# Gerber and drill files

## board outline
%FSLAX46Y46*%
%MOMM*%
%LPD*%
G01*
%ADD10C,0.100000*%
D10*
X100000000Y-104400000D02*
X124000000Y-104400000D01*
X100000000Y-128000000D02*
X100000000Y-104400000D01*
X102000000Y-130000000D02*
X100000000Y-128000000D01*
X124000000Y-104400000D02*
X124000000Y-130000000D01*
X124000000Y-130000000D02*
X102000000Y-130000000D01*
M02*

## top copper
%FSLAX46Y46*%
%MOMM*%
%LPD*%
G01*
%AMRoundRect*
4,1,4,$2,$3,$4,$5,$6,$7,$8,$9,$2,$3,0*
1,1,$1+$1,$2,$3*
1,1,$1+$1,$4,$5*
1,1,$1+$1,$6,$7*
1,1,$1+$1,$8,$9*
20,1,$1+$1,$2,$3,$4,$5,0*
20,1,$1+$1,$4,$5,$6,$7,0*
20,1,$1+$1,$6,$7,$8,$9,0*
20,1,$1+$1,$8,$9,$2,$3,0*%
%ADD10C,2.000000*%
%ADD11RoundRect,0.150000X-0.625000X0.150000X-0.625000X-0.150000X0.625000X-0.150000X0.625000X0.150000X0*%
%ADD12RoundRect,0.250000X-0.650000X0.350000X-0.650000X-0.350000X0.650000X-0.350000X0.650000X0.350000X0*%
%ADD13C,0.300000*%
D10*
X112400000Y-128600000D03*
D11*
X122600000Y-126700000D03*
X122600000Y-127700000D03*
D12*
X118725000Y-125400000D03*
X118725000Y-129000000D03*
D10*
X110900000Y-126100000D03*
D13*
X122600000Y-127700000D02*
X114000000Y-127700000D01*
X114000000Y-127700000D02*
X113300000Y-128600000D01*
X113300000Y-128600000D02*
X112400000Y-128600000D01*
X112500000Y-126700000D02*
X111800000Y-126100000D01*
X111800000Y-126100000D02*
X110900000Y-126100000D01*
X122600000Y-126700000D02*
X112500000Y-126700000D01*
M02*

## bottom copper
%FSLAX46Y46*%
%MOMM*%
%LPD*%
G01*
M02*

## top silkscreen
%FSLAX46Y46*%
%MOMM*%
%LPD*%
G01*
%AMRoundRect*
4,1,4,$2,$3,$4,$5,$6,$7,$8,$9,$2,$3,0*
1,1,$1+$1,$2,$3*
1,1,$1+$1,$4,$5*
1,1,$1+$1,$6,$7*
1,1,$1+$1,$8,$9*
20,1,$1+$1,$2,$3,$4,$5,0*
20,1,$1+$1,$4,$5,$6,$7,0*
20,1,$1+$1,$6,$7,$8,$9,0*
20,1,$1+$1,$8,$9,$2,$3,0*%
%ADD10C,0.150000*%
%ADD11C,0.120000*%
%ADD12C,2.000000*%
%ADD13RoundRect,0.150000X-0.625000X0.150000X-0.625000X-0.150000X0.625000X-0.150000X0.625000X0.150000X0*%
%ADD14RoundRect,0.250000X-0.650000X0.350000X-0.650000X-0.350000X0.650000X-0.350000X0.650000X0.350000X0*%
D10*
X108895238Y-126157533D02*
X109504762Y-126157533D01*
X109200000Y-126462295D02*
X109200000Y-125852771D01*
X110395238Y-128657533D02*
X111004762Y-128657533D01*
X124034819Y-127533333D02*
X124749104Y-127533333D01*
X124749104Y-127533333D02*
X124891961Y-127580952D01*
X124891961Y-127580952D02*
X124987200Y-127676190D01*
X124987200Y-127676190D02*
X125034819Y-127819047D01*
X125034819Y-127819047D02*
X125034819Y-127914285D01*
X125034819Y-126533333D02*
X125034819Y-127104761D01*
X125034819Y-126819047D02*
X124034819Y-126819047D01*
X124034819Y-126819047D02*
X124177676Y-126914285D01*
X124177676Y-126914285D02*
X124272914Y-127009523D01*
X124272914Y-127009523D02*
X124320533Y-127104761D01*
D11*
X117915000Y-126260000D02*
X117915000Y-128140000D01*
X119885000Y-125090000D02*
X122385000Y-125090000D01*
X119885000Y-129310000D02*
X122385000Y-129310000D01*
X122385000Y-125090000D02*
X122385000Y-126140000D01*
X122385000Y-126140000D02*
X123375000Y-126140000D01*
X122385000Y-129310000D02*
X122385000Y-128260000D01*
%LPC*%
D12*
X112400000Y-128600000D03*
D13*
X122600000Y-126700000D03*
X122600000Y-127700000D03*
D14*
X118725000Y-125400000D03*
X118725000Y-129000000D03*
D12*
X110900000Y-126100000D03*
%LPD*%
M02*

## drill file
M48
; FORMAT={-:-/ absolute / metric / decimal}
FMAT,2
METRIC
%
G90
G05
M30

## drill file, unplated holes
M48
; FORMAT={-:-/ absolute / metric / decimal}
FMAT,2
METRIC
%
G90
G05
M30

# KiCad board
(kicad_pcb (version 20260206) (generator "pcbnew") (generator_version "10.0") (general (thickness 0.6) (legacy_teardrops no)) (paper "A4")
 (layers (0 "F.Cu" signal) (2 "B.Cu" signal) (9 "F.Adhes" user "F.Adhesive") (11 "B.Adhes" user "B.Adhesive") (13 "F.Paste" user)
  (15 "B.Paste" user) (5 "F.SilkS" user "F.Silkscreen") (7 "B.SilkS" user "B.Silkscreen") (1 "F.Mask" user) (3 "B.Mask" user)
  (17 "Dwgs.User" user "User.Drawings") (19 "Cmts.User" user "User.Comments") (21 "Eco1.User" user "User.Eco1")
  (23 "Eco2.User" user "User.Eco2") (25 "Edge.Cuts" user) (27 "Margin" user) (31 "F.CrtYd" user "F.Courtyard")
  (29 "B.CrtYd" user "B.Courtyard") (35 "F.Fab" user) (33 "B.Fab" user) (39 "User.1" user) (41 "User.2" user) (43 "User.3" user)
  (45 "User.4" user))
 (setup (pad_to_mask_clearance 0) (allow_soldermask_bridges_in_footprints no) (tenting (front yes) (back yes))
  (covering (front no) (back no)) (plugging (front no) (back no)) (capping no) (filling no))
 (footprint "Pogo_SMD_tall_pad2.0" (layer "F.Cu") (at 112.4 128.6)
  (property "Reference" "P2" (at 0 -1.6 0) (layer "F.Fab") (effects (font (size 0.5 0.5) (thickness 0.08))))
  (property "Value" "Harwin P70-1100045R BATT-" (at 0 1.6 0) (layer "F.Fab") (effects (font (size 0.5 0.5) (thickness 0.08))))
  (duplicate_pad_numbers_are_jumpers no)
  (pad "1" smd circle (at 0 0) (size 2 2) (layers "F.Cu" "F.Mask" "F.Paste") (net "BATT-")))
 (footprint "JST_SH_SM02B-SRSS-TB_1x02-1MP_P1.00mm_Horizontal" (layer "F.Cu") (at 120.6 127.2 -90)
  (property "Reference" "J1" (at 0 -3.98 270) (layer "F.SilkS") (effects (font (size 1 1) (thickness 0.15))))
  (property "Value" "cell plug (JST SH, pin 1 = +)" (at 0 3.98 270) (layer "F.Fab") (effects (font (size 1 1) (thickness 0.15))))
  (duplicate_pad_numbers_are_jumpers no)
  (fp_line (start -0.94 2.685) (end 0.94 2.685) (stroke (width 0.12) (type solid)) (layer "F.SilkS"))
  (fp_line (start -2.11 0.715) (end -2.11 -1.785) (stroke (width 0.12) (type solid)) (layer "F.SilkS"))
  (fp_line (start 2.11 0.715) (end 2.11 -1.785) (stroke (width 0.12) (type solid)) (layer "F.SilkS"))
  (fp_line (start -2.11 -1.785) (end -1.06 -1.785) (stroke (width 0.12) (type solid)) (layer "F.SilkS"))
  (fp_line (start -1.06 -1.785) (end -1.06 -2.775) (stroke (width 0.12) (type solid)) (layer "F.SilkS"))
  (fp_line (start 2.11 -1.785) (end 1.06 -1.785) (stroke (width 0.12) (type solid)) (layer "F.SilkS"))
  (pad "1" smd roundrect (at -0.5 -2 270) (size 0.6 1.55) (layers "F.Cu" "F.Mask" "F.Paste") (roundrect_rratio 0.25) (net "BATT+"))
  (pad "2" smd roundrect (at 0.5 -2 270) (size 0.6 1.55) (layers "F.Cu" "F.Mask" "F.Paste") (roundrect_rratio 0.25) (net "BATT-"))
  (pad "MP" smd roundrect (at -1.8 1.875 270) (size 1.2 1.8) (layers "F.Cu" "F.Mask" "F.Paste") (roundrect_rratio 0.208333))
  (pad "MP" smd roundrect (at 1.8 1.875 270) (size 1.2 1.8) (layers "F.Cu" "F.Mask" "F.Paste") (roundrect_rratio 0.208333)))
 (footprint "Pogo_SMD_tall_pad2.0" (layer "F.Cu") (at 110.9 126.1)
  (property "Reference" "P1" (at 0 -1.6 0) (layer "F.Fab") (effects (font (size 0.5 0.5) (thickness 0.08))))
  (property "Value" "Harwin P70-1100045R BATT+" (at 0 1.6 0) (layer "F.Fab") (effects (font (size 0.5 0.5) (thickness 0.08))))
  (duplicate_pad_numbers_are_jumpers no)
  (pad "1" smd circle (at 0 0) (size 2 2) (layers "F.Cu" "F.Mask" "F.Paste") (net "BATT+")))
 (gr_line (start 100 104.4) (end 124 104.4) (stroke (width 0.1) (type default)) (layer "Edge.Cuts"))
 (gr_line (start 100 128) (end 100 104.4) (stroke (width 0.1) (type default)) (layer "Edge.Cuts"))
 (gr_line (start 102 130) (end 100 128) (stroke (width 0.1) (type default)) (layer "Edge.Cuts"))
 (gr_line (start 124 104.4) (end 124 130) (stroke (width 0.1) (type default)) (layer "Edge.Cuts"))
 (gr_line (start 124 130) (end 102 130) (stroke (width 0.1) (type default)) (layer "Edge.Cuts"))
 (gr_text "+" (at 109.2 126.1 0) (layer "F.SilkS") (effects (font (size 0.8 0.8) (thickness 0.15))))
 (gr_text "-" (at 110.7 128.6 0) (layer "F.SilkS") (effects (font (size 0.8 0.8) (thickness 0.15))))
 (segment (start 122.6 127.7) (end 114 127.7) (width 0.3) (layer "F.Cu") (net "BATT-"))
 (segment (start 114 127.7) (end 113.3 128.6) (width 0.3) (layer "F.Cu") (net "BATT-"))
 (segment (start 113.3 128.6) (end 112.4 128.6) (width 0.3) (layer "F.Cu") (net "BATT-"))
 (segment (start 112.5 126.7) (end 111.8 126.1) (width 0.3) (layer "F.Cu") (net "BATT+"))
 (segment (start 111.8 126.1) (end 110.9 126.1) (width 0.3) (layer "F.Cu") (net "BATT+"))
 (segment (start 122.6 126.7) (end 112.5 126.7) (width 0.3) (layer "F.Cu") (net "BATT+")))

